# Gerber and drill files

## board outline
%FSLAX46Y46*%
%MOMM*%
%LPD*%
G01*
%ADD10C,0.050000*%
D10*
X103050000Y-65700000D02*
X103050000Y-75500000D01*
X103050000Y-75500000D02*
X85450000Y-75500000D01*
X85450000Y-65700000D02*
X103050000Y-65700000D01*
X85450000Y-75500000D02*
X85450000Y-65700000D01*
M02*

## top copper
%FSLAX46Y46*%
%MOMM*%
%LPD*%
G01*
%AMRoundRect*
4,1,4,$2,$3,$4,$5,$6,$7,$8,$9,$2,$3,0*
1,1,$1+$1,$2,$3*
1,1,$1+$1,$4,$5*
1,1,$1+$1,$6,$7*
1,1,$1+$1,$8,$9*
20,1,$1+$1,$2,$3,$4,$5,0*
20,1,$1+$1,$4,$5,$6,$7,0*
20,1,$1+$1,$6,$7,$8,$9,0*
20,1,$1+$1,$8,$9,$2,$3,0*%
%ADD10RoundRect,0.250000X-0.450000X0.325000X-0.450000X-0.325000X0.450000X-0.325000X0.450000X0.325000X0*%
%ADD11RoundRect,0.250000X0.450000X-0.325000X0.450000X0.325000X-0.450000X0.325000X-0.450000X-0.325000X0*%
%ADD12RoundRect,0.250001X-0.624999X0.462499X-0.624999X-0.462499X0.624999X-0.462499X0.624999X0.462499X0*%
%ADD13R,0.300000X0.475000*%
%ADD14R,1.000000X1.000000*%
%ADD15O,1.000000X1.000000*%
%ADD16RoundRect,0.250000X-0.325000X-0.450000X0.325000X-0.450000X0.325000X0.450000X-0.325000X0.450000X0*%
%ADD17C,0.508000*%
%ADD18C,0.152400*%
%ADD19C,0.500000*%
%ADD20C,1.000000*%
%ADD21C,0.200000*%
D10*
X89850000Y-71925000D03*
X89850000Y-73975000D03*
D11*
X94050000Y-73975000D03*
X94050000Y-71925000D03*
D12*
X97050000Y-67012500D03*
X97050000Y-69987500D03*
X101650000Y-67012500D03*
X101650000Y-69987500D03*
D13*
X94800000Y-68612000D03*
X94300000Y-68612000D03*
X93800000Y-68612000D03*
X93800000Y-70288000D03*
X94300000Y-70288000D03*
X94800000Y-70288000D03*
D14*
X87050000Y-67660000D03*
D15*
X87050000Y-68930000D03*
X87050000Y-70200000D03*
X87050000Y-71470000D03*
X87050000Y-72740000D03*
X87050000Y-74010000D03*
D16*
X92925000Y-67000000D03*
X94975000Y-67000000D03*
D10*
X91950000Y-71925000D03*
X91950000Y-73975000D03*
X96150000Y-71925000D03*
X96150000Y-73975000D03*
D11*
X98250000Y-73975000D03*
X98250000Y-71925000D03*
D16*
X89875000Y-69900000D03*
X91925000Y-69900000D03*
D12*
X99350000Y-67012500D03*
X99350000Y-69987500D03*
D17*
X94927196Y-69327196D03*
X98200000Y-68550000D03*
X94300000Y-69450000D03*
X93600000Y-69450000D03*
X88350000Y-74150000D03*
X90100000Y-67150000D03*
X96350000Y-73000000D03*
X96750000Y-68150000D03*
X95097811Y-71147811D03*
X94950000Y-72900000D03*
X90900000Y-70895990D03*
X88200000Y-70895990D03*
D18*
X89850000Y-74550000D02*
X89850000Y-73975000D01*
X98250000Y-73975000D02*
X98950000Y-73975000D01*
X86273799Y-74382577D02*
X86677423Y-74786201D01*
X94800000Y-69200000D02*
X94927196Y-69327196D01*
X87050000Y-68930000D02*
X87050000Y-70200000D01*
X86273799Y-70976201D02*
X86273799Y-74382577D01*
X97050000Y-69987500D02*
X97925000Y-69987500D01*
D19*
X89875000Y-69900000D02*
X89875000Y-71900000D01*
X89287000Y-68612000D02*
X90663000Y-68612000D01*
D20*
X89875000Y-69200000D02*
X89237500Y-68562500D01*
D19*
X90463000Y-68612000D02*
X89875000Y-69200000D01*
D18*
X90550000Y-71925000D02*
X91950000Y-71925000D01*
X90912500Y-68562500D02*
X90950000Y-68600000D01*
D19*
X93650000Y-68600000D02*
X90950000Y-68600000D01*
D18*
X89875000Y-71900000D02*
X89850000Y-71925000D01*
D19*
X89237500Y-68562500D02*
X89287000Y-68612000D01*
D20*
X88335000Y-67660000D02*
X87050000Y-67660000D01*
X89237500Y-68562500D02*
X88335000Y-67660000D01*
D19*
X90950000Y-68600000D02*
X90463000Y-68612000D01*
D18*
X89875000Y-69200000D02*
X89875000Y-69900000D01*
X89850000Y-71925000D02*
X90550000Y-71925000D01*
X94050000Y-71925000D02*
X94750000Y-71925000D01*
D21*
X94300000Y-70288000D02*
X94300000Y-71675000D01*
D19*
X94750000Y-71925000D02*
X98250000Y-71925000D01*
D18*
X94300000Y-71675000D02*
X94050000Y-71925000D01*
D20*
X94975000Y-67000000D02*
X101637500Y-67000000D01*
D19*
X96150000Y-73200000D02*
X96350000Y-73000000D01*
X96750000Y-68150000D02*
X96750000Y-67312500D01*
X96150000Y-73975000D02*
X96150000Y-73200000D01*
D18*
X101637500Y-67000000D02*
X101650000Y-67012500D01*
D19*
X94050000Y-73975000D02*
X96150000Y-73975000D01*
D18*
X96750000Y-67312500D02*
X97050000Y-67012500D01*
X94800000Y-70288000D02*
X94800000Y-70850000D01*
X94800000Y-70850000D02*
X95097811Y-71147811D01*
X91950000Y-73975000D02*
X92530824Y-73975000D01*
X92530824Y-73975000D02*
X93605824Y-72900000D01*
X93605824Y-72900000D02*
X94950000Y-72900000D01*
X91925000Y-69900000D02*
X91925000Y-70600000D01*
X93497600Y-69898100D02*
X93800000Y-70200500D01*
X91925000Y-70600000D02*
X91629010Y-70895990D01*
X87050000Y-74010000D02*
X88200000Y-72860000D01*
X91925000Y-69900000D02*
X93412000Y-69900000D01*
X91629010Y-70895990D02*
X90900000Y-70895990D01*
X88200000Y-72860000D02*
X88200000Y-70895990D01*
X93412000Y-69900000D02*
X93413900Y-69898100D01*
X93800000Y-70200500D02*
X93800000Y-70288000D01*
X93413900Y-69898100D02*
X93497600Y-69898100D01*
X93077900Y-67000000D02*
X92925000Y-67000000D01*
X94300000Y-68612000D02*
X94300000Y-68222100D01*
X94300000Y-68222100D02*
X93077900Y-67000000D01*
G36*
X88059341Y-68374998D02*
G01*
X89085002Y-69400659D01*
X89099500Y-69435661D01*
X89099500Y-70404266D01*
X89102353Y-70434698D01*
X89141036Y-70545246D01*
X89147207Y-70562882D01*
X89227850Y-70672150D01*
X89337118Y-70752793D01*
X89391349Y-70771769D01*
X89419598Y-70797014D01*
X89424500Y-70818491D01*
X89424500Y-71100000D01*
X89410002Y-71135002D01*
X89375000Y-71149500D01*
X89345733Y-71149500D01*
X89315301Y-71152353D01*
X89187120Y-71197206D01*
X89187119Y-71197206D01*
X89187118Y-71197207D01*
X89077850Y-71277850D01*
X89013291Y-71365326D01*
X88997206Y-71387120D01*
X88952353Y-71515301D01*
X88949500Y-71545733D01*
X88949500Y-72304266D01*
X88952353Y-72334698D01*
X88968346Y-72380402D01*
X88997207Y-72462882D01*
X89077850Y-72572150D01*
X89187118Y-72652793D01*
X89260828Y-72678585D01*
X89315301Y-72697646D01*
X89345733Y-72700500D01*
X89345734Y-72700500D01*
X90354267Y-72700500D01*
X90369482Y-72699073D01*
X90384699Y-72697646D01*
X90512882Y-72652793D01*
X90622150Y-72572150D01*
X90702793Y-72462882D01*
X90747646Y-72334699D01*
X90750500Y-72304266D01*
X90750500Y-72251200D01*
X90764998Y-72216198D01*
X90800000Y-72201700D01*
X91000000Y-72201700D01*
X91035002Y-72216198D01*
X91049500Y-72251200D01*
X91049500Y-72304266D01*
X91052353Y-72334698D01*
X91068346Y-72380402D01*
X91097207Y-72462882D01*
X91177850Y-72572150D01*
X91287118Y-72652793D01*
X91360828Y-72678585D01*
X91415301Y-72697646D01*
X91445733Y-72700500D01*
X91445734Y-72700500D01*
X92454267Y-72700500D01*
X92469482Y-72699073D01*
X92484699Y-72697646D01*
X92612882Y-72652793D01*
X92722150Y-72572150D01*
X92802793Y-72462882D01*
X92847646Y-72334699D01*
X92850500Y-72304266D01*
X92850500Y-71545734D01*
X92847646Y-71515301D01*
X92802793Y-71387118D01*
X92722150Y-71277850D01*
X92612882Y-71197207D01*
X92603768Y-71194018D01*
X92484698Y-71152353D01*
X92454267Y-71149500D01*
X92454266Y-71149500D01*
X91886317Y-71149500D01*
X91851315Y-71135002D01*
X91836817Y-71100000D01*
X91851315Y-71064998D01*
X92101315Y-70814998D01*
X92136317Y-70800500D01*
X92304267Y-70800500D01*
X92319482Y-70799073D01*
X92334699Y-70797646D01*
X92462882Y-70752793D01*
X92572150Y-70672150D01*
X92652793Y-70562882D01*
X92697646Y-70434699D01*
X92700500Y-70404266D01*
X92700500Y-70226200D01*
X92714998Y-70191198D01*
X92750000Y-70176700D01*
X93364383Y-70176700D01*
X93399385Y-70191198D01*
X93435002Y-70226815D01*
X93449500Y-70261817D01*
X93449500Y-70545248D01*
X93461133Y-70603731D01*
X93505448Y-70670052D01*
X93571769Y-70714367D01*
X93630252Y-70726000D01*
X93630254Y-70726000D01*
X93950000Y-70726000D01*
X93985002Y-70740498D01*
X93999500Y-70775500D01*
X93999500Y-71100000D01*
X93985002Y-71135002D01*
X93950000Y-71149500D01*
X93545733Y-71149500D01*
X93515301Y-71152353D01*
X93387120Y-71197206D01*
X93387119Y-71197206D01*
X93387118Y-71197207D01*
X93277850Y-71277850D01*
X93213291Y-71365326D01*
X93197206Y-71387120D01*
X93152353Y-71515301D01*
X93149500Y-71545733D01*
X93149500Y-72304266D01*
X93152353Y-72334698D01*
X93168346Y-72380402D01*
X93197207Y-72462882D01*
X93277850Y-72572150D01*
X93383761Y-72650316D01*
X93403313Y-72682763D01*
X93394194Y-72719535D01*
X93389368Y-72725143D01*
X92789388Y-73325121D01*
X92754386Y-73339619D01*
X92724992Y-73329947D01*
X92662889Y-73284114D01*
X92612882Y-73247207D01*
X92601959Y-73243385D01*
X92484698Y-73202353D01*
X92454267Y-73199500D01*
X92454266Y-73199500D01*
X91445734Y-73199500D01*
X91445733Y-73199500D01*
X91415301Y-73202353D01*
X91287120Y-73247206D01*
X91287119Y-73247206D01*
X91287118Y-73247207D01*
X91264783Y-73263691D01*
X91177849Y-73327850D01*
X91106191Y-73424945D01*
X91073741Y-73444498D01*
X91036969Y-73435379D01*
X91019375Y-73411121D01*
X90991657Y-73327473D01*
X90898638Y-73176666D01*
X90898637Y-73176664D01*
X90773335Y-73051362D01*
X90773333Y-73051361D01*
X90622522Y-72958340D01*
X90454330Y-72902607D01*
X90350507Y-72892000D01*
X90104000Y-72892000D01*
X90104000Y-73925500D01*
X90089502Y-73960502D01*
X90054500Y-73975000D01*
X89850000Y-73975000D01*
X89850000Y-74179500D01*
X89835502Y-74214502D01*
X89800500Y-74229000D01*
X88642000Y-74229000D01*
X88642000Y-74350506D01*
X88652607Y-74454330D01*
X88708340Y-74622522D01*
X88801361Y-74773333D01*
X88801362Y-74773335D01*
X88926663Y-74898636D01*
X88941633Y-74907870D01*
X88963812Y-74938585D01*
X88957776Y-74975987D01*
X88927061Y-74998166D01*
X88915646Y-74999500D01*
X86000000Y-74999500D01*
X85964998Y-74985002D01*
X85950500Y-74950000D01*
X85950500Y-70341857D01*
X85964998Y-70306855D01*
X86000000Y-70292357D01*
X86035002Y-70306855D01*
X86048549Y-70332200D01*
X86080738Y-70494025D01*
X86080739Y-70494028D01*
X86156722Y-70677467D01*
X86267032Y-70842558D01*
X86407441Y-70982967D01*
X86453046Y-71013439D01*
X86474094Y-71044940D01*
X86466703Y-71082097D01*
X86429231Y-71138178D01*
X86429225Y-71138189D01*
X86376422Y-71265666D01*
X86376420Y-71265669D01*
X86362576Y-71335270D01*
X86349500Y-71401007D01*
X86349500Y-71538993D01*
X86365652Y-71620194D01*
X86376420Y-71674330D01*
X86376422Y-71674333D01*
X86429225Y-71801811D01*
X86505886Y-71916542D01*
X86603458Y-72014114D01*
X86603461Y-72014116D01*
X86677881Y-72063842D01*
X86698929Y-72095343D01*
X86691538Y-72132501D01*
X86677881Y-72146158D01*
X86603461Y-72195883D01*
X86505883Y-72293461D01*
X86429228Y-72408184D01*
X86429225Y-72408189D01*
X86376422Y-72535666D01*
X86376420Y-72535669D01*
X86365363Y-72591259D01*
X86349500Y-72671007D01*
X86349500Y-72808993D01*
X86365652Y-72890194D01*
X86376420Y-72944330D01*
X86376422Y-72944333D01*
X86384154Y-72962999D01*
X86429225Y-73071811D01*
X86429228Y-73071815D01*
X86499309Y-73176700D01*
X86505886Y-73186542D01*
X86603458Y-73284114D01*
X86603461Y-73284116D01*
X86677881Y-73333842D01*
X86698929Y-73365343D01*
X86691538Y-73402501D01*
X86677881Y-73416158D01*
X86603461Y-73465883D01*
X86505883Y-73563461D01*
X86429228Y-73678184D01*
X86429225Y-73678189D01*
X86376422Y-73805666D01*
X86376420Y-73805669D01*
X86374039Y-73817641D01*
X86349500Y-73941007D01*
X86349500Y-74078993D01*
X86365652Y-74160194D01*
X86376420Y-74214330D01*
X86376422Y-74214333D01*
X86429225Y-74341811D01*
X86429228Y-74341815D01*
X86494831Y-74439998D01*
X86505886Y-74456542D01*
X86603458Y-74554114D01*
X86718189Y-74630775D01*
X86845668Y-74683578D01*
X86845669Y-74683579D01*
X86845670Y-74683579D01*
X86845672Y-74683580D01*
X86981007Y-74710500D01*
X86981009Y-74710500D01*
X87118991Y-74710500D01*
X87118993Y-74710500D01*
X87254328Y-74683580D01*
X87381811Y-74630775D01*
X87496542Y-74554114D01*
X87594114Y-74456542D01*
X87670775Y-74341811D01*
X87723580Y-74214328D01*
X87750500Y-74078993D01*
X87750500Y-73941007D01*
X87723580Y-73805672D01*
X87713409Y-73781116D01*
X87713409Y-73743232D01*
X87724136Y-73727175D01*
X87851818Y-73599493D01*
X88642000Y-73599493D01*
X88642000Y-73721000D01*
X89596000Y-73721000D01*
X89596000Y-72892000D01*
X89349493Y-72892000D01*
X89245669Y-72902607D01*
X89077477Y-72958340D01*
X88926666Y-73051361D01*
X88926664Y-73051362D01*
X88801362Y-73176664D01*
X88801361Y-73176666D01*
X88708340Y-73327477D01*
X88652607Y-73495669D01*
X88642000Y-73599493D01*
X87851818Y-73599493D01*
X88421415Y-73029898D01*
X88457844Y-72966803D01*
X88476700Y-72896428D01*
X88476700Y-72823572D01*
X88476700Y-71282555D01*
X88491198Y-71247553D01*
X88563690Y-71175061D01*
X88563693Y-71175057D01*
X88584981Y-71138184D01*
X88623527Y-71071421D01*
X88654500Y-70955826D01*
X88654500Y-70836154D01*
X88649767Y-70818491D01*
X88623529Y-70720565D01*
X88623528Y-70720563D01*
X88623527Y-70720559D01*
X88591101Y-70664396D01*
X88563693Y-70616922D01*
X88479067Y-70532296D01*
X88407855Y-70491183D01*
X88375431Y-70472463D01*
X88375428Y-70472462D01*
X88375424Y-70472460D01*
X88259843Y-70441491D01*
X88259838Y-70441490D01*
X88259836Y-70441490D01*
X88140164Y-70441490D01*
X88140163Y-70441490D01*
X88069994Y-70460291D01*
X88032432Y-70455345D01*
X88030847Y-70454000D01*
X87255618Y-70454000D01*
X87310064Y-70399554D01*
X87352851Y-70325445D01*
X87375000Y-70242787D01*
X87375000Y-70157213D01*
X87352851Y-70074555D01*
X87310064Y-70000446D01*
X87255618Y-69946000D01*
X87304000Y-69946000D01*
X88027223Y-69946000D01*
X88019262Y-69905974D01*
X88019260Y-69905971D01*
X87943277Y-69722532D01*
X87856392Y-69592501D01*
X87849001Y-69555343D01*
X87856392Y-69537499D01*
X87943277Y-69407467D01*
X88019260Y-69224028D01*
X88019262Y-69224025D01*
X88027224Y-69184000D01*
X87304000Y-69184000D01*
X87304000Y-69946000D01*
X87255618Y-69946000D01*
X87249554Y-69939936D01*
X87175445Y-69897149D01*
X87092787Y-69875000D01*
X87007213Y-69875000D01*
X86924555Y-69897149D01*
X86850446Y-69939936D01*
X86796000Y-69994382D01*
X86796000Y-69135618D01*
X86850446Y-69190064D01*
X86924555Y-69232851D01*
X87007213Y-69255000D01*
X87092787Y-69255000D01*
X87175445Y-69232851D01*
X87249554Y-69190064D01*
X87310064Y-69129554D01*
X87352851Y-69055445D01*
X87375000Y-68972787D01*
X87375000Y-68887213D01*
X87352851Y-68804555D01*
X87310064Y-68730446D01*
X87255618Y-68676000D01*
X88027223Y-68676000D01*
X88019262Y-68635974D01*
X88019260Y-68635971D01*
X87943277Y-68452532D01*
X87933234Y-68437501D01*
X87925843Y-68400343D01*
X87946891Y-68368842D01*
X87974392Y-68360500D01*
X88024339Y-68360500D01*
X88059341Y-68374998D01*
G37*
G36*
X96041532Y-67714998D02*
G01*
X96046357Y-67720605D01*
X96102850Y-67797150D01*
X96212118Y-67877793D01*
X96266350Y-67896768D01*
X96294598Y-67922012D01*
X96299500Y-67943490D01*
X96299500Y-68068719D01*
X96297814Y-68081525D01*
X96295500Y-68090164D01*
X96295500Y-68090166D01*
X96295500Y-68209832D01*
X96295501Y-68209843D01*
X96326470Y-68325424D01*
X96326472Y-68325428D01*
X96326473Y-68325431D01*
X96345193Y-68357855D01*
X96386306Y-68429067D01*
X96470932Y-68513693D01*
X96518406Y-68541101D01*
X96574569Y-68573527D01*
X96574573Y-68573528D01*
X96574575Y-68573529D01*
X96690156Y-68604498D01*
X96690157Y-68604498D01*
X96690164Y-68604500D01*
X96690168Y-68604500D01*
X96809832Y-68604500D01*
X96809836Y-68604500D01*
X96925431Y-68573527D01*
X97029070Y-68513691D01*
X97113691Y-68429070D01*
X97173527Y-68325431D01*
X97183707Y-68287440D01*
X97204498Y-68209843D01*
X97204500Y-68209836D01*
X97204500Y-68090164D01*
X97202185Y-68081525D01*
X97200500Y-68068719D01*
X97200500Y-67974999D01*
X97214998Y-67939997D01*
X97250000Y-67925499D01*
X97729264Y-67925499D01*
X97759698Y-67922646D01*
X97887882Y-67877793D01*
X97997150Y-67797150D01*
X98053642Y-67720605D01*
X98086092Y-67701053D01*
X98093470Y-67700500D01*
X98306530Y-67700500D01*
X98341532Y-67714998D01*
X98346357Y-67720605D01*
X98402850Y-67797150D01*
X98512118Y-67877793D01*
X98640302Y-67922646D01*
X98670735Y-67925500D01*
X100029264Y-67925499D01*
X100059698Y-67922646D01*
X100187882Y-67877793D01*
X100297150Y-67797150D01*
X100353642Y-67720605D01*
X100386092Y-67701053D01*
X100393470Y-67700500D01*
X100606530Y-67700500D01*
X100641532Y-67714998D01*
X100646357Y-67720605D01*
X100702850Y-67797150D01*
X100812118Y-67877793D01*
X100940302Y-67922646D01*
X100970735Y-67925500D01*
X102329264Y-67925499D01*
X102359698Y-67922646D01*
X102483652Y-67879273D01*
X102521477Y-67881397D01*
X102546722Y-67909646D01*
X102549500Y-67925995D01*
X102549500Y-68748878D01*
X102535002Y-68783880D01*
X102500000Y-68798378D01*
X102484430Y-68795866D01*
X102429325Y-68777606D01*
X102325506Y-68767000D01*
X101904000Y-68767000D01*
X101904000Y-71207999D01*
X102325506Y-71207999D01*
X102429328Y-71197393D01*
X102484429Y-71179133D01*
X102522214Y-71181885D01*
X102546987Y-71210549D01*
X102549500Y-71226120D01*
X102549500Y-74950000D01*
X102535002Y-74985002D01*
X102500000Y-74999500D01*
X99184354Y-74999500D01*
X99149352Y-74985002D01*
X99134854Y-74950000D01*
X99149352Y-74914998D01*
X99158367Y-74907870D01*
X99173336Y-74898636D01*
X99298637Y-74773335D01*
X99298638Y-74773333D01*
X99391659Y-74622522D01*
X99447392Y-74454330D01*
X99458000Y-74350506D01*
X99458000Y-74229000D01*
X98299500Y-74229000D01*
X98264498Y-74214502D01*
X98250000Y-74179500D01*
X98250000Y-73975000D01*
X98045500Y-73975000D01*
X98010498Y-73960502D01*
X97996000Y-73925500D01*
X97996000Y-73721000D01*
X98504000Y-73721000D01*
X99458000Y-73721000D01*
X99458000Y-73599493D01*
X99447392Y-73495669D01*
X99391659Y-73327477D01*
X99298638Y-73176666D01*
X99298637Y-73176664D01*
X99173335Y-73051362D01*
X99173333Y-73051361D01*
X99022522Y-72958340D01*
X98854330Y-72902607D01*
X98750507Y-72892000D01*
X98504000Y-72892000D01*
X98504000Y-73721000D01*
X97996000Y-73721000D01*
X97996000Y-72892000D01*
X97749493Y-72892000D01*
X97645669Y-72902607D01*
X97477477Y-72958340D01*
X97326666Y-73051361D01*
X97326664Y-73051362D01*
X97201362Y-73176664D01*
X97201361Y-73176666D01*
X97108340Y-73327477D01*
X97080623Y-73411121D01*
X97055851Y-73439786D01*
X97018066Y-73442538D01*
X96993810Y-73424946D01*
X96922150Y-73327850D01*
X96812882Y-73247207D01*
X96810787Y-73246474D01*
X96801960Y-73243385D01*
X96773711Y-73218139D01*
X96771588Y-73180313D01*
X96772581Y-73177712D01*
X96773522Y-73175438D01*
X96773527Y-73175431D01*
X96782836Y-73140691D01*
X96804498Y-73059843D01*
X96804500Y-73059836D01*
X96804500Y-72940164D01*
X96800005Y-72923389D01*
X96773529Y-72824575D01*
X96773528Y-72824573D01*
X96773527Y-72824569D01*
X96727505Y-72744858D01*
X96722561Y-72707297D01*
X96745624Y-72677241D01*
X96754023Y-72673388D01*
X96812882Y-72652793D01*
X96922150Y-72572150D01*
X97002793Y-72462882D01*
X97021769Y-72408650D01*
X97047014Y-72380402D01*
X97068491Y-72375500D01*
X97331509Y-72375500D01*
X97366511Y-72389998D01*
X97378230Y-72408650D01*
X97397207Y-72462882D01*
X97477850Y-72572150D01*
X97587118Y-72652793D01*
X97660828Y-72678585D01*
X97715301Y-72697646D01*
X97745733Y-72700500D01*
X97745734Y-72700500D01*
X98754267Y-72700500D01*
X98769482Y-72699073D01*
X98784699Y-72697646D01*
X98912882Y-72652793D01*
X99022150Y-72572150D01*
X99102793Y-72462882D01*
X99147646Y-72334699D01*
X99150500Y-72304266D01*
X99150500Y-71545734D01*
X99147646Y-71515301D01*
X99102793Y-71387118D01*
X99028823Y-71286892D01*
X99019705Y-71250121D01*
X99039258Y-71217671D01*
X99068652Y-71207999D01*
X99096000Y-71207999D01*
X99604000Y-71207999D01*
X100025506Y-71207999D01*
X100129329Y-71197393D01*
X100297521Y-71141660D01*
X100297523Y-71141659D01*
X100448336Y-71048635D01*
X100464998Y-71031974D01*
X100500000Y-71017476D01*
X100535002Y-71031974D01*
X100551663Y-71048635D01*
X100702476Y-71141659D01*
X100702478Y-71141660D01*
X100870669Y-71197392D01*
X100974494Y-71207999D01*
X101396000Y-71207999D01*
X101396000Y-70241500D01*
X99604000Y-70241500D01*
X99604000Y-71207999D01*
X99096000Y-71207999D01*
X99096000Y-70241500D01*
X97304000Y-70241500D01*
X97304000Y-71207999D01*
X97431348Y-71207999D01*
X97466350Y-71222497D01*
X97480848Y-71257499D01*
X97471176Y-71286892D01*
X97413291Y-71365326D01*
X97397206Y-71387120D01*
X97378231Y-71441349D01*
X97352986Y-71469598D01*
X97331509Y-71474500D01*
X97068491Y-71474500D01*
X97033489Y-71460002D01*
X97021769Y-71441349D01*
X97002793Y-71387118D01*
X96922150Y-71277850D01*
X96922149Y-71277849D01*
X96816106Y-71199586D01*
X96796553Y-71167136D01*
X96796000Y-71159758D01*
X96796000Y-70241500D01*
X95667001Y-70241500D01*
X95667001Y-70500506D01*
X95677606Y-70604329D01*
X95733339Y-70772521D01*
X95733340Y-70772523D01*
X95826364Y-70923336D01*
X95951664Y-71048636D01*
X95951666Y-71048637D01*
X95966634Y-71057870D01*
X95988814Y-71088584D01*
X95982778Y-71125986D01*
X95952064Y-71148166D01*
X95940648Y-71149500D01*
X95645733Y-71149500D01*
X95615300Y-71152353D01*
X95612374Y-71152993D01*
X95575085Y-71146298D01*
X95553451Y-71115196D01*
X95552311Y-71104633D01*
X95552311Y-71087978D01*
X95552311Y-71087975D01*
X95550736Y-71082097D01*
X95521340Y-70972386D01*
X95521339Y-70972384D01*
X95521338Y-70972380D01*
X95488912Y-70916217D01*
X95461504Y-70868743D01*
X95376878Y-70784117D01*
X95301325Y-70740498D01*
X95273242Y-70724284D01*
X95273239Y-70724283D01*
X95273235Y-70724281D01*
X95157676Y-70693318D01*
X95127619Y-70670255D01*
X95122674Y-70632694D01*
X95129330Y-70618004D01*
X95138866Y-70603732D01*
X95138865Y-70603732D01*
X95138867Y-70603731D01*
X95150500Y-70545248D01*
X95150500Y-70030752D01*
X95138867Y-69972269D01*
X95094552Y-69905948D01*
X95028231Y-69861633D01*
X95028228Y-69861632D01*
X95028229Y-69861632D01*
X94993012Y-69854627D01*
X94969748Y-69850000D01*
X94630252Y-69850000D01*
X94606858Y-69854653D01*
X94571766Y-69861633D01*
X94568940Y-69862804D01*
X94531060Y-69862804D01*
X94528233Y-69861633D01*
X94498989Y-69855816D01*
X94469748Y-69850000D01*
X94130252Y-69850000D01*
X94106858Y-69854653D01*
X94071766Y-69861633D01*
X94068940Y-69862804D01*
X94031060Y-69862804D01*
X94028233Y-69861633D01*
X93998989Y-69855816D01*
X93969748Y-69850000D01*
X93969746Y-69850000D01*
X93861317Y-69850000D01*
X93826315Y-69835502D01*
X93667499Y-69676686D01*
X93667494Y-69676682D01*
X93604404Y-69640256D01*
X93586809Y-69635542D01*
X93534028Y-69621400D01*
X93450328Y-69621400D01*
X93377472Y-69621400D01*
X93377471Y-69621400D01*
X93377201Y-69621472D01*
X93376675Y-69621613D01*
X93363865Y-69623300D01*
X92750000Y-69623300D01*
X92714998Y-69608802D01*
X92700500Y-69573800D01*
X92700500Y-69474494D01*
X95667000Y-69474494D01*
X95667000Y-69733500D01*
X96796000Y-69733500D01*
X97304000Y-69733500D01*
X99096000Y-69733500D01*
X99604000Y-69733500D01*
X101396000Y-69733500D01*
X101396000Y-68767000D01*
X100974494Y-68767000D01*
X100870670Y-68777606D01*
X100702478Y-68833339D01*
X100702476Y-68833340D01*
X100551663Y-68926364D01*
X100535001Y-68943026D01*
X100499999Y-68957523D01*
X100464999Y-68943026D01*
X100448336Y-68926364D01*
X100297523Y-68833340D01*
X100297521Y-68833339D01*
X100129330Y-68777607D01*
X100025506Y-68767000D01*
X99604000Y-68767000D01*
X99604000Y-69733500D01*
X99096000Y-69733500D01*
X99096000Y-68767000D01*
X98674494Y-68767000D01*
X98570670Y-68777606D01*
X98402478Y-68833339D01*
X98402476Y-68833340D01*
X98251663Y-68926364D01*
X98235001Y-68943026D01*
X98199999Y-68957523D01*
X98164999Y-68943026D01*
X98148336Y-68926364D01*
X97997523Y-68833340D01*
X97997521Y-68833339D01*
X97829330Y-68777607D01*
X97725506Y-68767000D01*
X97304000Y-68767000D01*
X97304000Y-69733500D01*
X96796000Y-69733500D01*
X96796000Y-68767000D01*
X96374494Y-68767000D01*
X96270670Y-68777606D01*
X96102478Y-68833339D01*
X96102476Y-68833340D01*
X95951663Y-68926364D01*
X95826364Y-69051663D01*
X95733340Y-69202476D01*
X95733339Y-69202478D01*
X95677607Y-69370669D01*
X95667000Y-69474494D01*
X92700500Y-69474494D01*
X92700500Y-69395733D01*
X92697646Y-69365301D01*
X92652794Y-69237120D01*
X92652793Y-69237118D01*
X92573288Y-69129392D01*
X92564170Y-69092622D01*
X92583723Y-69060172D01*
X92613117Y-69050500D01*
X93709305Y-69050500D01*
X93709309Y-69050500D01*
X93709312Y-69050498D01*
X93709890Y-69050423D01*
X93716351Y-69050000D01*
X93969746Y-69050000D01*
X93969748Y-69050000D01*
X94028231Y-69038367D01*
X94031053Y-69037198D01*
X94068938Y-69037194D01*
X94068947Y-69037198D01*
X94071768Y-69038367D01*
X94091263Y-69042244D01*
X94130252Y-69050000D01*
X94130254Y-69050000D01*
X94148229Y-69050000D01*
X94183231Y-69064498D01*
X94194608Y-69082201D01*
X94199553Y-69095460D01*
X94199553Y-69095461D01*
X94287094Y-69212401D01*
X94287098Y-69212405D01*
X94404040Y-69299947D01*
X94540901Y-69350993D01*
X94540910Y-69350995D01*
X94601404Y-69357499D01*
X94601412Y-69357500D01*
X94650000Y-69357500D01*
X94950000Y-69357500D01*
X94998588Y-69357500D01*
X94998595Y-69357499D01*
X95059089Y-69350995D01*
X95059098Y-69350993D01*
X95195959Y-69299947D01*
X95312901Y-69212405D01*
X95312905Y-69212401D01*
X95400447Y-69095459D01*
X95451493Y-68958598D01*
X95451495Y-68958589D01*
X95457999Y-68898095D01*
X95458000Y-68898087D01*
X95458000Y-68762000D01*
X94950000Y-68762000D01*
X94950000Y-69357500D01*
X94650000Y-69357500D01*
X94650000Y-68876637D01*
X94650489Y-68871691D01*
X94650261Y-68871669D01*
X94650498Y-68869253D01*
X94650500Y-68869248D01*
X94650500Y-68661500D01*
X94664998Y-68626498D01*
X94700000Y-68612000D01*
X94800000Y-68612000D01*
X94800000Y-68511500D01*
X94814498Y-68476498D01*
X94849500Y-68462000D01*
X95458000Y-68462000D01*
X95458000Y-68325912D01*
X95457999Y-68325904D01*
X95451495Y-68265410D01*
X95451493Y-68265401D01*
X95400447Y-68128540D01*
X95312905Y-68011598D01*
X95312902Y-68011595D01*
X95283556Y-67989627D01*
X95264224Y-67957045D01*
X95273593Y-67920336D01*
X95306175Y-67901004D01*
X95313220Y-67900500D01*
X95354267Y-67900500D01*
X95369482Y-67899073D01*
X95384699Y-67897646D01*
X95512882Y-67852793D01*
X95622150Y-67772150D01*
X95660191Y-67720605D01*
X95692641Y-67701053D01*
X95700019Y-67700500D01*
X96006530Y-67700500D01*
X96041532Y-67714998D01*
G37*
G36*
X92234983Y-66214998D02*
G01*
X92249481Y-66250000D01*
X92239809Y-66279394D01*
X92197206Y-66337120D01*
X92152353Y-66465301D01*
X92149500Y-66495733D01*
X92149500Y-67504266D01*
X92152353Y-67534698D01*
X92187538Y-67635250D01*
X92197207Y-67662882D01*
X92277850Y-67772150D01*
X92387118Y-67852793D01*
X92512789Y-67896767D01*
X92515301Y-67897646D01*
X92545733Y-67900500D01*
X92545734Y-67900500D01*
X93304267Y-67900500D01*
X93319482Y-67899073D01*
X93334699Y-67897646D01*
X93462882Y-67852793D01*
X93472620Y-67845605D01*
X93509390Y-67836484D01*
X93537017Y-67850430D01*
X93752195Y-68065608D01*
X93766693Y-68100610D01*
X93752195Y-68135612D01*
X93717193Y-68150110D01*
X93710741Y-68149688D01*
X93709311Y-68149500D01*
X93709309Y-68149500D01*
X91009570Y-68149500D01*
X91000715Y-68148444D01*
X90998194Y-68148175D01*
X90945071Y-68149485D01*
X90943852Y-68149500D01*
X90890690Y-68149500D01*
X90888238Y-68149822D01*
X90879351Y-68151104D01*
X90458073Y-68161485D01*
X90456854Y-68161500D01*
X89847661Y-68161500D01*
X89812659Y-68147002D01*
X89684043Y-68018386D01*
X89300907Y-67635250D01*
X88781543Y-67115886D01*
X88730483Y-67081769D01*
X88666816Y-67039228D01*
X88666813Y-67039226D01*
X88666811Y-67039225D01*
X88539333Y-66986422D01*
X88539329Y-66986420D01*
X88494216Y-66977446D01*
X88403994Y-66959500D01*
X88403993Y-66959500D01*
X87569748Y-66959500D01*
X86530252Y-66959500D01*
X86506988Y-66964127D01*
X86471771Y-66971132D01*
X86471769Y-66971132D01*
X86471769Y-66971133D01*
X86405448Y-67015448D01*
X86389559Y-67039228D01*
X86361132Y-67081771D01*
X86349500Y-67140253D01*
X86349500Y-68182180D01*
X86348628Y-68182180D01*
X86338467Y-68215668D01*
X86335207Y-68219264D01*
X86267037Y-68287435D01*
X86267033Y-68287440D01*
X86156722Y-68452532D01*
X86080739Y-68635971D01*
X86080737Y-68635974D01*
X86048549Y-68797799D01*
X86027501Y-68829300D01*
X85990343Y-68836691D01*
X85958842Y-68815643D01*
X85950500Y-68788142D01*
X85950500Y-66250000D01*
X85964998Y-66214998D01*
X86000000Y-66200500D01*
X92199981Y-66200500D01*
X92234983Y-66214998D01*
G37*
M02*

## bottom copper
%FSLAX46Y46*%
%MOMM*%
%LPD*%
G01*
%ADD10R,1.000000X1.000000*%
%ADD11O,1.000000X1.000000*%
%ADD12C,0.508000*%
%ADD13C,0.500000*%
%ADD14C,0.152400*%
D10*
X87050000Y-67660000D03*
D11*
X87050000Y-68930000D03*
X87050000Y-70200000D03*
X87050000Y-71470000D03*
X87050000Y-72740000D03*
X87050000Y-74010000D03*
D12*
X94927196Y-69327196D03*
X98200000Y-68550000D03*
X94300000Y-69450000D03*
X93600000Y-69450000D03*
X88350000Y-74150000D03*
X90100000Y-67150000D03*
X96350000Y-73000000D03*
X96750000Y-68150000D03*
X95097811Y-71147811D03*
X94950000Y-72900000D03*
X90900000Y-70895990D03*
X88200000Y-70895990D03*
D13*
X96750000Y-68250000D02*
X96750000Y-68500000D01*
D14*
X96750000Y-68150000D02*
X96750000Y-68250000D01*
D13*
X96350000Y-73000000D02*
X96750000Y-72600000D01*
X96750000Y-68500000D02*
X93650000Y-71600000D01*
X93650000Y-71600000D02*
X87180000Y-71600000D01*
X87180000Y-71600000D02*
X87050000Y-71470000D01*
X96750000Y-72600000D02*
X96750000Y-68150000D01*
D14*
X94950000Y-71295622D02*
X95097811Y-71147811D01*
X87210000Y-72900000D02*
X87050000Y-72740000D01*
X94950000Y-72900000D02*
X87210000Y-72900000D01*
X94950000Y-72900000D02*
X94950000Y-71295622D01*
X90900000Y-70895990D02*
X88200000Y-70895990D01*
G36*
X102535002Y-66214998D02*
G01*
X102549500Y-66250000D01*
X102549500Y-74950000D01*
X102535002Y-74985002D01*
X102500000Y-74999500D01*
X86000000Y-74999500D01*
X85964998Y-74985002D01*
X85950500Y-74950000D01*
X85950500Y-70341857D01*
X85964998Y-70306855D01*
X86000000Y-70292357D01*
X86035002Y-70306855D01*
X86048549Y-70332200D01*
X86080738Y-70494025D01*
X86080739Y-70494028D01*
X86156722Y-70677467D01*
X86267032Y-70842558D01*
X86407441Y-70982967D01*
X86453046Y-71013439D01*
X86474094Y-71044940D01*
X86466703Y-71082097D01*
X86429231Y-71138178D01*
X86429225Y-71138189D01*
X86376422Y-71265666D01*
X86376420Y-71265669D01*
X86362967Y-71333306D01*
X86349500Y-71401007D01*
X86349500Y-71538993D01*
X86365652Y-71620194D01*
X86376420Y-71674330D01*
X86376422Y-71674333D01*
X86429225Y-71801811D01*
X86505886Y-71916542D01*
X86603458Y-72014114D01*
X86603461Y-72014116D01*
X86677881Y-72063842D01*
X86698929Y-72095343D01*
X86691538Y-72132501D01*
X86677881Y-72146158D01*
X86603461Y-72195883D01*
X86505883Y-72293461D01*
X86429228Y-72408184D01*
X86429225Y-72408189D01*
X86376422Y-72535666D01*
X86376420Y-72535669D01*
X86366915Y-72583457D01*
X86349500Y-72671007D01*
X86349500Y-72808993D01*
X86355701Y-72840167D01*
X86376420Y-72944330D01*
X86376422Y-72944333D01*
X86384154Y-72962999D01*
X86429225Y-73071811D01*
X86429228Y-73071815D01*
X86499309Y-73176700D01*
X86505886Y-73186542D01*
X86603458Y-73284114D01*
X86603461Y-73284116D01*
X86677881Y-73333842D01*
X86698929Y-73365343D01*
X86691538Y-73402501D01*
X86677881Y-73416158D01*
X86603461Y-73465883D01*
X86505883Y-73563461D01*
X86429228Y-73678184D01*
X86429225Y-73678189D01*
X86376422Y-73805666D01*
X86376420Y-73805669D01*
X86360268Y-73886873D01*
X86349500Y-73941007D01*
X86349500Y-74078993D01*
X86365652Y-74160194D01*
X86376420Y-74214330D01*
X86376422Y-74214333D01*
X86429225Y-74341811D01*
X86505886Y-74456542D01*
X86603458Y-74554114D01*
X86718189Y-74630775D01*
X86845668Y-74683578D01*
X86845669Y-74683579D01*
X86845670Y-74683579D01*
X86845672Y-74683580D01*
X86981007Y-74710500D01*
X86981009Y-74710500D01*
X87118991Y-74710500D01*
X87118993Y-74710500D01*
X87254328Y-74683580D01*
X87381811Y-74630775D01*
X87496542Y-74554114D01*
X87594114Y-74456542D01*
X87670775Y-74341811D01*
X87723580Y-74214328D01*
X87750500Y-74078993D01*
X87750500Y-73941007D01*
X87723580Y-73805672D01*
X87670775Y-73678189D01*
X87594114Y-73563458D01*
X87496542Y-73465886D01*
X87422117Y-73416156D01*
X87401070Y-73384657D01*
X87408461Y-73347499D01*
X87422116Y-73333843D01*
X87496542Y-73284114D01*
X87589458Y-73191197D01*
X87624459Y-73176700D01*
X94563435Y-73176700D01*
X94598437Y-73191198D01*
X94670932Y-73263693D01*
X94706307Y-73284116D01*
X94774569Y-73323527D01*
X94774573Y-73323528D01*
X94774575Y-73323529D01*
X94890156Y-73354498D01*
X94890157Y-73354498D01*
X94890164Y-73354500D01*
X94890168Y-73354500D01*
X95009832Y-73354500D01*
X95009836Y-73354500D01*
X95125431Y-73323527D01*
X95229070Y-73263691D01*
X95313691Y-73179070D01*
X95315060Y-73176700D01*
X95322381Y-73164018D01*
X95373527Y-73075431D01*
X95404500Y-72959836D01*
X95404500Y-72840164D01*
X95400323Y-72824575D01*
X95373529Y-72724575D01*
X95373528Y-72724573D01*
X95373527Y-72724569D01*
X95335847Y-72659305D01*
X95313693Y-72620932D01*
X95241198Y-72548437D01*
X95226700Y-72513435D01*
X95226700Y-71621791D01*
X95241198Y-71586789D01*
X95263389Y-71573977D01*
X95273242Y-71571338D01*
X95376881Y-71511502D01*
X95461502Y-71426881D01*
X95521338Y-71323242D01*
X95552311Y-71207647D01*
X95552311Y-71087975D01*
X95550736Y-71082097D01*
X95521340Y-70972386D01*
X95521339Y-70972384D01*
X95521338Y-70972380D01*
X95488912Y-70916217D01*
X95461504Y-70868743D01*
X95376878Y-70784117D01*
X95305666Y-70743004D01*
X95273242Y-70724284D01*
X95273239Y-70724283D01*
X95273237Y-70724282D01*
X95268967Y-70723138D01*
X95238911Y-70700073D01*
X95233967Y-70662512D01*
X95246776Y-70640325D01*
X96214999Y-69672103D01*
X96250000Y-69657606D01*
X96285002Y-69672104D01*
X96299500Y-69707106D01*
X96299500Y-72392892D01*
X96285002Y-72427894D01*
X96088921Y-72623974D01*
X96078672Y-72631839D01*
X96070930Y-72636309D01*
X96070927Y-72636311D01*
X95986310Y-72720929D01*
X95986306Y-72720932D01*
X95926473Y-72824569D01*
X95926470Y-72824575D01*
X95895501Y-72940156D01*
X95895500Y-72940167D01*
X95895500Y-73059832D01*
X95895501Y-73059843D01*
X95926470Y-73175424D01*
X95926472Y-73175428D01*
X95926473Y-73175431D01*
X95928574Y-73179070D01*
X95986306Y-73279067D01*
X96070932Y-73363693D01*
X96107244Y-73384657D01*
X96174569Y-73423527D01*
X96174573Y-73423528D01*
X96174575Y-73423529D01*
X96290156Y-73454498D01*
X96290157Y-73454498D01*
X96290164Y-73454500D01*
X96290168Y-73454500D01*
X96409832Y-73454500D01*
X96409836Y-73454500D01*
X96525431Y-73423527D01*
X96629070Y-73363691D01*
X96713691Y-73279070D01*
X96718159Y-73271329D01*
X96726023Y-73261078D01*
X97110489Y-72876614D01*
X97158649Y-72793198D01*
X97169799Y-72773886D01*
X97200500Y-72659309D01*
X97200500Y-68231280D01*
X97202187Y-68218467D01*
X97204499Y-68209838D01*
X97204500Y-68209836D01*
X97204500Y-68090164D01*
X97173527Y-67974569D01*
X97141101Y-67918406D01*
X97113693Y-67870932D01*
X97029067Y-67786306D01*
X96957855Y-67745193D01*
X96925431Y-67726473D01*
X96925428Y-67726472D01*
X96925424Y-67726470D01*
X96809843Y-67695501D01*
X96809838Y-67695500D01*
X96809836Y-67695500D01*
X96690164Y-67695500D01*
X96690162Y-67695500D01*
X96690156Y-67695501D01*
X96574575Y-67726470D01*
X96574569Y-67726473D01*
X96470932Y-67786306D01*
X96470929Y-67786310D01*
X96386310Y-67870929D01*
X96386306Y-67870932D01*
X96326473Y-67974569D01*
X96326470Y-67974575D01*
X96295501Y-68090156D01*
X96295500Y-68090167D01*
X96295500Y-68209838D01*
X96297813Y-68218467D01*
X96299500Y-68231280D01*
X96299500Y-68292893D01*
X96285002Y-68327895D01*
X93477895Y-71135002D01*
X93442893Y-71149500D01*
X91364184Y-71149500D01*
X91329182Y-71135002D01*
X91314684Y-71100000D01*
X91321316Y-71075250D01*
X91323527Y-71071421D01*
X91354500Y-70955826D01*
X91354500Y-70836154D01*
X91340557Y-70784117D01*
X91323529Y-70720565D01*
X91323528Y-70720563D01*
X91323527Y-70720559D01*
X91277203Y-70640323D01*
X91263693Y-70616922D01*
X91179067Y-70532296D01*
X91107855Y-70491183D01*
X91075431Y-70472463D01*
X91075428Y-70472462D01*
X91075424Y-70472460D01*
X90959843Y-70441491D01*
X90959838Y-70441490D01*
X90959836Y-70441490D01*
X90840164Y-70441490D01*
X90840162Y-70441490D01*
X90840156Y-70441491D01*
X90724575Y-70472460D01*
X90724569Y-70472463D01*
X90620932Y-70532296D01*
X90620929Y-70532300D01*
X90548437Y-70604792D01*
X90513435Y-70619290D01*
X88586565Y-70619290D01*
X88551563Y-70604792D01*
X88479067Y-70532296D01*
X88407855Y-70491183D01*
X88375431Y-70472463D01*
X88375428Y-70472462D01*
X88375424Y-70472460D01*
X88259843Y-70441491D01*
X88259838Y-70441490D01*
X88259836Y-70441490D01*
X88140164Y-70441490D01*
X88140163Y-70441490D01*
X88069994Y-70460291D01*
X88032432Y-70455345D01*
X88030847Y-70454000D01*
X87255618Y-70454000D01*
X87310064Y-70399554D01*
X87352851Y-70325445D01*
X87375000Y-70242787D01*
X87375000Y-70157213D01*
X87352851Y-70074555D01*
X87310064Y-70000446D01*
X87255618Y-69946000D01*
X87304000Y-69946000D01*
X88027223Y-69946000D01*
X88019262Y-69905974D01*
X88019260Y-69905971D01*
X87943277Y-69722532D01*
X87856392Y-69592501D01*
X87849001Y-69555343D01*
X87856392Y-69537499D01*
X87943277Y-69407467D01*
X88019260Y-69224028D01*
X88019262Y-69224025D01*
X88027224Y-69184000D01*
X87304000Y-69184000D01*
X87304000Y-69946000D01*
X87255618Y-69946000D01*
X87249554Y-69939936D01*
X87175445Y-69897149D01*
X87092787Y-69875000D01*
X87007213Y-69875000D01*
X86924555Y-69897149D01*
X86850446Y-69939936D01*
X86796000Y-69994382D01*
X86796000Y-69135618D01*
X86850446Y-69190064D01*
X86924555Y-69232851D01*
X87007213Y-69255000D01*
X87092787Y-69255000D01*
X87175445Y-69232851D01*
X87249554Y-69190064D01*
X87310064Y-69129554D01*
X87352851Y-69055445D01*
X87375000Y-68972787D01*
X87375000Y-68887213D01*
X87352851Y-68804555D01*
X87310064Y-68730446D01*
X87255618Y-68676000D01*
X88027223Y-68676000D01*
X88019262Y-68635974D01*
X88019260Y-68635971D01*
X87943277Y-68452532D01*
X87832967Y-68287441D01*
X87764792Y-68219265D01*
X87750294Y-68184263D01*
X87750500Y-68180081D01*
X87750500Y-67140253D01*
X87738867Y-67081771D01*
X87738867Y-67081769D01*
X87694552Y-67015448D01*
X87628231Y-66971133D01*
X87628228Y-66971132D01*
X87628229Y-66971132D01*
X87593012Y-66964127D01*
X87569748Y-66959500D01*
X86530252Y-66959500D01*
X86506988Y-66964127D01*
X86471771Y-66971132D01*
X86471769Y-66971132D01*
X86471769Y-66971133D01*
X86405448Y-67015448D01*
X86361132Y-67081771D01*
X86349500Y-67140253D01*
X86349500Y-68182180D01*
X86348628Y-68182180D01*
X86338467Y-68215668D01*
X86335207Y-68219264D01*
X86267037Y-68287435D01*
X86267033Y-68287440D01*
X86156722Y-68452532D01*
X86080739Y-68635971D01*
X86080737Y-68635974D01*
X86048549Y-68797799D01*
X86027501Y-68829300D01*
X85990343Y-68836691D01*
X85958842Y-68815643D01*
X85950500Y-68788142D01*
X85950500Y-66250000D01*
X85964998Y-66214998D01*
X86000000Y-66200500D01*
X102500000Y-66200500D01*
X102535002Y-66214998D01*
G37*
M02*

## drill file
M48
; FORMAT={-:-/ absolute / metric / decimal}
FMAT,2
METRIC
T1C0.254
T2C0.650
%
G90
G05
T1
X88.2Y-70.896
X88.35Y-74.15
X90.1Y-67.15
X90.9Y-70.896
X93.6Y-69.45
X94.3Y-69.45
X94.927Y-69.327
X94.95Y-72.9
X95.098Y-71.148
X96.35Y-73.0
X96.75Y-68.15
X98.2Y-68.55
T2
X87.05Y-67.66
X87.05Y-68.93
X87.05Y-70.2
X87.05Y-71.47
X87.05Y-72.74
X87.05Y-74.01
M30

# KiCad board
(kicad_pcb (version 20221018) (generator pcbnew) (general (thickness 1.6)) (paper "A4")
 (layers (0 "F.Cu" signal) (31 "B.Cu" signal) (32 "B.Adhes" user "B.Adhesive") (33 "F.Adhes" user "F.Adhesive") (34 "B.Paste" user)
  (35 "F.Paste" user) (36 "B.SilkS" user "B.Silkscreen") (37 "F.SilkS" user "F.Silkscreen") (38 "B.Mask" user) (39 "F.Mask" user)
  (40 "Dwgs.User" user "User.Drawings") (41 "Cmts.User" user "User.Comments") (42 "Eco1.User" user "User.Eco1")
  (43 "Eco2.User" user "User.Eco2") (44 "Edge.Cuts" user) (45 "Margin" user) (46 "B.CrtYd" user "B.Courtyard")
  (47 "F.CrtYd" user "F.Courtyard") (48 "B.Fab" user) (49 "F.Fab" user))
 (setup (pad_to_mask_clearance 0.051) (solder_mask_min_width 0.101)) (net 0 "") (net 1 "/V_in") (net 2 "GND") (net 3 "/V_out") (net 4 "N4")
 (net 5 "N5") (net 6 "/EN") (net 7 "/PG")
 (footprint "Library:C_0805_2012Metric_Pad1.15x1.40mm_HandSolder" (layer "F.Cu") (at 89.85 72.95 -90)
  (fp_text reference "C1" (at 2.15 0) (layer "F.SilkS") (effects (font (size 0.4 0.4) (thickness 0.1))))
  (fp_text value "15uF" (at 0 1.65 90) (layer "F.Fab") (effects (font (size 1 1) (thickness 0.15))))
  (pad "1" smd roundrect (at -1.025 0 270) (size 1.15 1.4) (layers "F.Cu" "F.Paste" "F.Mask") (roundrect_rratio 0.217391) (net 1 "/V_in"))
  (pad "2" smd roundrect (at 1.025 0 270) (size 1.15 1.4) (layers "F.Cu" "F.Paste" "F.Mask") (roundrect_rratio 0.217391) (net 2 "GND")))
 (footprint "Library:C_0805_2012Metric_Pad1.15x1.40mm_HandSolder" (layer "F.Cu") (at 94.05 72.95 90)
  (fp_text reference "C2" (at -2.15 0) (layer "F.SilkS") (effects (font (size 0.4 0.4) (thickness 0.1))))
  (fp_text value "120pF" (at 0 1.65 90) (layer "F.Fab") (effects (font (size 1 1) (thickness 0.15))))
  (pad "1" smd roundrect (at -1.025 0 90) (size 1.15 1.4) (layers "F.Cu" "F.Paste" "F.Mask") (roundrect_rratio 0.217391) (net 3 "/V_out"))
  (pad "2" smd roundrect (at 1.025 0 90) (size 1.15 1.4) (layers "F.Cu" "F.Paste" "F.Mask") (roundrect_rratio 0.217391) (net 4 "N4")))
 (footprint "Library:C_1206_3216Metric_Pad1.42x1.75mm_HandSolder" (layer "F.Cu") (at 97.05 68.5 -90)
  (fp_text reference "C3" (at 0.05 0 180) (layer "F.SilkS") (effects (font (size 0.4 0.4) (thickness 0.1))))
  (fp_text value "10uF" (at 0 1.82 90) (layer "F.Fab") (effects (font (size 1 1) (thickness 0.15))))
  (pad "1" smd roundrect (at -1.4875 0 270) (size 1.425 1.75) (layers "F.Cu" "F.Paste" "F.Mask") (roundrect_rratio 0.175439)
   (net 3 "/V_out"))
  (pad "2" smd roundrect (at 1.4875 0 270) (size 1.425 1.75) (layers "F.Cu" "F.Paste" "F.Mask") (roundrect_rratio 0.175439) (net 2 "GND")))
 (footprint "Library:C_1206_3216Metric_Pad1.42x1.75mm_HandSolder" (layer "F.Cu") (at 101.65 68.5 -90)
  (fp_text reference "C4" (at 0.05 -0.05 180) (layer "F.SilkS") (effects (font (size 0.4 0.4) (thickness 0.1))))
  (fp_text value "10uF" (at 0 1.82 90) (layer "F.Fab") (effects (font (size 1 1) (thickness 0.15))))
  (pad "1" smd roundrect (at -1.4875 0 270) (size 1.425 1.75) (layers "F.Cu" "F.Paste" "F.Mask") (roundrect_rratio 0.175439)
   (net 3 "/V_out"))
  (pad "2" smd roundrect (at 1.4875 0 270) (size 1.425 1.75) (layers "F.Cu" "F.Paste" "F.Mask") (roundrect_rratio 0.175439) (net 2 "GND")))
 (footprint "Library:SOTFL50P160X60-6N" (layer "F.Cu") (at 94.3 69.45 -90)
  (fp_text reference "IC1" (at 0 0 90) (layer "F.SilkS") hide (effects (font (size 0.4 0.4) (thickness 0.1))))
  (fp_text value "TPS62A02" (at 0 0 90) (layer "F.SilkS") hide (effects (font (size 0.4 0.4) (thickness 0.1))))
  (pad "1" smd rect (at -0.838 -0.5) (size 0.3 0.475) (layers "F.Cu" "F.Paste" "F.Mask") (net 2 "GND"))
  (pad "2" smd rect (at -0.838 0) (size 0.3 0.475) (layers "F.Cu" "F.Paste" "F.Mask") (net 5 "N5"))
  (pad "3" smd rect (at -0.838 0.5) (size 0.3 0.475) (layers "F.Cu" "F.Paste" "F.Mask") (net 1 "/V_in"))
  (pad "4" smd rect (at 0.838 0.5) (size 0.3 0.475) (layers "F.Cu" "F.Paste" "F.Mask") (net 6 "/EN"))
  (pad "5" smd rect (at 0.838 0) (size 0.3 0.475) (layers "F.Cu" "F.Paste" "F.Mask") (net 4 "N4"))
  (pad "6" smd rect (at 0.838 -0.5) (size 0.3 0.475) (layers "F.Cu" "F.Paste" "F.Mask") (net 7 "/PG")))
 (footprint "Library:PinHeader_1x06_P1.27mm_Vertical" (layer "F.Cu") (at 87.05 67.66)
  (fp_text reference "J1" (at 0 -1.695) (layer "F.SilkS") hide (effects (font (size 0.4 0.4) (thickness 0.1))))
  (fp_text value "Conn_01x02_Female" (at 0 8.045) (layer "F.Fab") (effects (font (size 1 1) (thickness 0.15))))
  (pad "1" thru_hole rect (at 0 0) (size 1 1) (drill 0.65) (layers "*.Cu" "*.Mask") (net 1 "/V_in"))
  (pad "2" thru_hole oval (at 0 1.27) (size 1 1) (drill 0.65) (layers "*.Cu" "*.Mask") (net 2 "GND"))
  (pad "3" thru_hole oval (at 0 2.54) (size 1 1) (drill 0.65) (layers "*.Cu" "*.Mask") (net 2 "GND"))
  (pad "4" thru_hole oval (at 0 3.81) (size 1 1) (drill 0.65) (layers "*.Cu" "*.Mask") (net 3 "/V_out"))
  (pad "5" thru_hole oval (at 0 5.08) (size 1 1) (drill 0.65) (layers "*.Cu" "*.Mask") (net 7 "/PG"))
  (pad "6" thru_hole oval (at 0 6.35) (size 1 1) (drill 0.65) (layers "*.Cu" "*.Mask") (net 6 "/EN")))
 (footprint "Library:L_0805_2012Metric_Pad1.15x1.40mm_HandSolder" (layer "F.Cu") (at 93.95 67)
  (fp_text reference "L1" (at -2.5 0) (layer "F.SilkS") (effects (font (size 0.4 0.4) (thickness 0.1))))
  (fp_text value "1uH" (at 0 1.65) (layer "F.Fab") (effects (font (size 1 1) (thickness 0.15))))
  (pad "1" smd roundrect (at -1.025 0) (size 1.15 1.4) (layers "F.Cu" "F.Paste" "F.Mask") (roundrect_rratio 0.217391) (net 5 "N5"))
  (pad "2" smd roundrect (at 1.025 0) (size 1.15 1.4) (layers "F.Cu" "F.Paste" "F.Mask") (roundrect_rratio 0.217391) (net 3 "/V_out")))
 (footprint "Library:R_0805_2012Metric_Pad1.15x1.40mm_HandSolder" (layer "F.Cu") (at 91.95 72.95 -90)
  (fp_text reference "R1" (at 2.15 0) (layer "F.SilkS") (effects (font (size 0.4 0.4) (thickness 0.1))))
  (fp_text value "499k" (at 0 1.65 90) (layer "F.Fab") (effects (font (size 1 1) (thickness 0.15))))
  (pad "1" smd roundrect (at -1.025 0 270) (size 1.15 1.4) (layers "F.Cu" "F.Paste" "F.Mask") (roundrect_rratio 0.217391) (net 1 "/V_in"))
  (pad "2" smd roundrect (at 1.025 0 270) (size 1.15 1.4) (layers "F.Cu" "F.Paste" "F.Mask") (roundrect_rratio 0.217391) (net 7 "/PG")))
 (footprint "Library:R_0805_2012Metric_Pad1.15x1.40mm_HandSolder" (layer "F.Cu") (at 96.15 72.95 -90)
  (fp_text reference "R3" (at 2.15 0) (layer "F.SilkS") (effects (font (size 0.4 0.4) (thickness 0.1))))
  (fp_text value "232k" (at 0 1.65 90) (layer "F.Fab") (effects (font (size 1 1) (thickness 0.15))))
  (pad "1" smd roundrect (at -1.025 0 270) (size 1.15 1.4) (layers "F.Cu" "F.Paste" "F.Mask") (roundrect_rratio 0.217391) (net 4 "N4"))
  (pad "2" smd roundrect (at 1.025 0 270) (size 1.15 1.4) (layers "F.Cu" "F.Paste" "F.Mask") (roundrect_rratio 0.217391) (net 3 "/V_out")))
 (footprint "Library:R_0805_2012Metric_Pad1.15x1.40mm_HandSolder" (layer "F.Cu") (at 98.25 72.95 90)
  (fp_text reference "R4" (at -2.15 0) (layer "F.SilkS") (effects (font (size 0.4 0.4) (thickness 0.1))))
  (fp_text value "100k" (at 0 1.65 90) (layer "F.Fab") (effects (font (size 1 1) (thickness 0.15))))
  (pad "1" smd roundrect (at -1.025 0 90) (size 1.15 1.4) (layers "F.Cu" "F.Paste" "F.Mask") (roundrect_rratio 0.217391) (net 2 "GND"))
  (pad "2" smd roundrect (at 1.025 0 90) (size 1.15 1.4) (layers "F.Cu" "F.Paste" "F.Mask") (roundrect_rratio 0.217391) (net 4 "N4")))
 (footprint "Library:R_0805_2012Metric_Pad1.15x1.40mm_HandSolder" (layer "F.Cu") (at 90.9 69.9)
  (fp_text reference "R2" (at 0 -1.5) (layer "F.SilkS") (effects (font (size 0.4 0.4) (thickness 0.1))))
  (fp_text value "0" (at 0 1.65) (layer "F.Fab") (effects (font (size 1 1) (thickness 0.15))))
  (pad "1" smd roundrect (at -1.025 0) (size 1.15 1.4) (layers "F.Cu" "F.Paste" "F.Mask") (roundrect_rratio 0.217391) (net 1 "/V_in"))
  (pad "2" smd roundrect (at 1.025 0) (size 1.15 1.4) (layers "F.Cu" "F.Paste" "F.Mask") (roundrect_rratio 0.217391) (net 6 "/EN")))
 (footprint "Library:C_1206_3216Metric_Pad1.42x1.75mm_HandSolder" (layer "F.Cu") (at 99.35 68.5 -90)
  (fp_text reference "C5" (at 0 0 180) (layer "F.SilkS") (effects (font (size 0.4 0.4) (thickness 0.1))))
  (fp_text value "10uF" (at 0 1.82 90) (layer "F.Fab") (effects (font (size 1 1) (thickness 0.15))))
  (pad "1" smd roundrect (at -1.4875 0 270) (size 1.425 1.75) (layers "F.Cu" "F.Paste" "F.Mask") (roundrect_rratio 0.175439)
   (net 3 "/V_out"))
  (pad "2" smd roundrect (at 1.4875 0 270) (size 1.425 1.75) (layers "F.Cu" "F.Paste" "F.Mask") (roundrect_rratio 0.175439) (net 2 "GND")))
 (gr_line (start 103.05 65.7) (end 103.05 75.5) (stroke (width 0.05) (type solid)) (layer "Edge.Cuts"))
 (gr_line (start 103.05 75.5) (end 85.45 75.5) (stroke (width 0.05) (type solid)) (layer "Edge.Cuts"))
 (gr_line (start 85.45 65.7) (end 103.05 65.7) (stroke (width 0.05) (type solid)) (layer "Edge.Cuts"))
 (gr_line (start 85.45 75.5) (end 85.45 65.7) (stroke (width 0.05) (type solid)) (layer "Edge.Cuts"))
 (segment (start 89.85 74.55) (end 89.85 73.975) (width 0.1524) (layer "F.Cu") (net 2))
 (segment (start 98.25 73.975) (end 98.95 73.975) (width 0.1524) (layer "F.Cu") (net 2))
 (segment (start 86.273799 74.382577) (end 86.677423 74.786201) (width 0.1524) (layer "F.Cu") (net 2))
 (segment (start 94.8 69.2) (end 94.927196 69.327196) (width 0.1524) (layer "F.Cu") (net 2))
 (segment (start 87.05 68.93) (end 87.05 70.2) (width 0.1524) (layer "F.Cu") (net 2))
 (segment (start 86.273799 70.976201) (end 86.273799 74.382577) (width 0.1524) (layer "F.Cu") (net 2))
 (segment (start 97.05 69.9875) (end 97.925 69.9875) (width 0.1524) (layer "F.Cu") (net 2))
 (via (at 94.927196 69.327196) (size 0.508) (drill 0.254) (layers "F.Cu" "B.Cu") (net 2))
 (via (at 98.2 68.55) (size 0.508) (drill 0.254) (layers "F.Cu" "B.Cu") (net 2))
 (via (at 94.3 69.45) (size 0.508) (drill 0.254) (layers "F.Cu" "B.Cu") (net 2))
 (via (at 93.6 69.45) (size 0.508) (drill 0.254) (layers "F.Cu" "B.Cu") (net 2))
 (via (at 88.35 74.15) (size 0.508) (drill 0.254) (layers "F.Cu" "B.Cu") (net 2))
 (via (at 90.1 67.15) (size 0.508) (drill 0.254) (layers "F.Cu" "B.Cu") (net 2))
 (segment (start 89.875 69.9) (end 89.875 71.9) (width 0.5) (layer "F.Cu") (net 1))
 (segment (start 89.287 68.612) (end 90.663 68.612) (width 0.5) (layer "F.Cu") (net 1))
 (segment (start 89.875 69.2) (end 89.2375 68.5625) (width 1) (layer "F.Cu") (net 1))
 (segment (start 90.463 68.612) (end 89.875 69.2) (width 0.5) (layer "F.Cu") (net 1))
 (segment (start 90.55 71.925) (end 91.95 71.925) (width 0.1524) (layer "F.Cu") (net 1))
 (segment (start 90.9125 68.5625) (end 90.95 68.6) (width 0.1524) (layer "F.Cu") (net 1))
 (segment (start 93.65 68.6) (end 90.95 68.6) (width 0.5) (layer "F.Cu") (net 1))
 (segment (start 89.875 71.9) (end 89.85 71.925) (width 0.1524) (layer "F.Cu") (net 1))
 (segment (start 89.2375 68.5625) (end 89.287 68.612) (width 0.5) (layer "F.Cu") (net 1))
 (segment (start 88.335 67.66) (end 87.05 67.66) (width 1) (layer "F.Cu") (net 1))
 (segment (start 89.2375 68.5625) (end 88.335 67.66) (width 1) (layer "F.Cu") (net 1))
 (segment (start 90.95 68.6) (end 90.463 68.612) (width 0.5) (layer "F.Cu") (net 1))
 (segment (start 89.875 69.2) (end 89.875 69.9) (width 0.1524) (layer "F.Cu") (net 1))
 (segment (start 89.85 71.925) (end 90.55 71.925) (width 0.1524) (layer "F.Cu") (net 1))
 (segment (start 94.05 71.925) (end 94.75 71.925) (width 0.1524) (layer "F.Cu") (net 4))
 (segment (start 94.3 70.288) (end 94.3 71.675) (width 0.2) (layer "F.Cu") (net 4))
 (segment (start 94.75 71.925) (end 98.25 71.925) (width 0.5) (layer "F.Cu") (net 4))
 (segment (start 94.3 71.675) (end 94.05 71.925) (width 0.1524) (layer "F.Cu") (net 4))
 (segment (start 94.975 67) (end 101.6375 67) (width 1) (layer "F.Cu") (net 3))
 (segment (start 96.15 73.2) (end 96.35 73) (width 0.5) (layer "F.Cu") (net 3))
 (segment (start 96.75 68.15) (end 96.75 67.3125) (width 0.5) (layer "F.Cu") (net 3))
 (segment (start 96.15 73.975) (end 96.15 73.2) (width 0.5) (layer "F.Cu") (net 3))
 (segment (start 101.6375 67) (end 101.65 67.0125) (width 0.1524) (layer "F.Cu") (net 3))
 (segment (start 94.05 73.975) (end 96.15 73.975) (width 0.5) (layer "F.Cu") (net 3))
 (segment (start 96.75 67.3125) (end 97.05 67.0125) (width 0.1524) (layer "F.Cu") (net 3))
 (via (at 96.35 73) (size 0.508) (drill 0.254) (layers "F.Cu" "B.Cu") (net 3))
 (via (at 96.75 68.15) (size 0.508) (drill 0.254) (layers "F.Cu" "B.Cu") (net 3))
 (segment (start 96.75 68.25) (end 96.75 68.5) (width 0.5) (layer "B.Cu") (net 3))
 (segment (start 96.75 68.15) (end 96.75 68.25) (width 0.1524) (layer "B.Cu") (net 3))
 (segment (start 96.35 73) (end 96.75 72.6) (width 0.5) (layer "B.Cu") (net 3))
 (segment (start 96.75 68.5) (end 93.65 71.6) (width 0.5) (layer "B.Cu") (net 3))
 (segment (start 93.65 71.6) (end 87.18 71.6) (width 0.5) (layer "B.Cu") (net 3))
 (segment (start 87.18 71.6) (end 87.05 71.47) (width 0.5) (layer "B.Cu") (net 3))
 (segment (start 96.75 72.6) (end 96.75 68.15) (width 0.5) (layer "B.Cu") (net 3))
 (segment (start 94.8 70.288) (end 94.8 70.85) (width 0.1524) (layer "F.Cu") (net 7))
 (segment (start 94.8 70.85) (end 95.097811 71.147811) (width 0.1524) (layer "F.Cu") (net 7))
 (segment (start 91.95 73.975) (end 92.530824 73.975) (width 0.1524) (layer "F.Cu") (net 7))
 (segment (start 92.530824 73.975) (end 93.605824 72.9) (width 0.1524) (layer "F.Cu") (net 7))
 (segment (start 93.605824 72.9) (end 94.95 72.9) (width 0.1524) (layer "F.Cu") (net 7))
 (via (at 95.097811 71.147811) (size 0.508) (drill 0.254) (layers "F.Cu" "B.Cu") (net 7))
 (via (at 94.95 72.9) (size 0.508) (drill 0.254) (layers "F.Cu" "B.Cu") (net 7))
 (segment (start 94.95 71.295622) (end 95.097811 71.147811) (width 0.1524) (layer "B.Cu") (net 7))
 (segment (start 87.21 72.9) (end 87.05 72.74) (width 0.1524) (layer "B.Cu") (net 7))
 (segment (start 94.95 72.9) (end 87.21 72.9) (width 0.1524) (layer "B.Cu") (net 7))
 (segment (start 94.95 72.9) (end 94.95 71.295622) (width 0.1524) (layer "B.Cu") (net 7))
 (segment (start 91.925 69.9) (end 91.925 70.6) (width 0.1524) (layer "F.Cu") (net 6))
 (segment (start 93.4976 69.8981) (end 93.8 70.2005) (width 0.1524) (layer "F.Cu") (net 6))
 (segment (start 91.925 70.6) (end 91.62901 70.89599) (width 0.1524) (layer "F.Cu") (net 6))
 (segment (start 87.05 74.01) (end 88.2 72.86) (width 0.1524) (layer "F.Cu") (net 6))
 (segment (start 91.925 69.9) (end 93.412 69.9) (width 0.1524) (layer "F.Cu") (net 6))
 (segment (start 91.62901 70.89599) (end 90.9 70.89599) (width 0.1524) (layer "F.Cu") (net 6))
 (segment (start 88.2 72.86) (end 88.2 70.89599) (width 0.1524) (layer "F.Cu") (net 6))
 (segment (start 93.412 69.9) (end 93.4139 69.8981) (width 0.1524) (layer "F.Cu") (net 6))
 (segment (start 93.8 70.2005) (end 93.8 70.288) (width 0.1524) (layer "F.Cu") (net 6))
 (segment (start 93.4139 69.8981) (end 93.4976 69.8981) (width 0.1524) (layer "F.Cu") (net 6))
 (via (at 90.9 70.89599) (size 0.508) (drill 0.254) (layers "F.Cu" "B.Cu") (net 6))
 (via (at 88.2 70.89599) (size 0.508) (drill 0.254) (layers "F.Cu" "B.Cu") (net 6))
 (segment (start 90.9 70.89599) (end 88.2 70.89599) (width 0.1524) (layer "B.Cu") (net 6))
 (segment (start 93.0779 67) (end 92.925 67) (width 0.1524) (layer "F.Cu") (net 5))
 (segment (start 94.3 68.612) (end 94.3 68.2221) (width 0.1524) (layer "F.Cu") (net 5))
 (segment (start 94.3 68.2221) (end 93.0779 67) (width 0.1524) (layer "F.Cu") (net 5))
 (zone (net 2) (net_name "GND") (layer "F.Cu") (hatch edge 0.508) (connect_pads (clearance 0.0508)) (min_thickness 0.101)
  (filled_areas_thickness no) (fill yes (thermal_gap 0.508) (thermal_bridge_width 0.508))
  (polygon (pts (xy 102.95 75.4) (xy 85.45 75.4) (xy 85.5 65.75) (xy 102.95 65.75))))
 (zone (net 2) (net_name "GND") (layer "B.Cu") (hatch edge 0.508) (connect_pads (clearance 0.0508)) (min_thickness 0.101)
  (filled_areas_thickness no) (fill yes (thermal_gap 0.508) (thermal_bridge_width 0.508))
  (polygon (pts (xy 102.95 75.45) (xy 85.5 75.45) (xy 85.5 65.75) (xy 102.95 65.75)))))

